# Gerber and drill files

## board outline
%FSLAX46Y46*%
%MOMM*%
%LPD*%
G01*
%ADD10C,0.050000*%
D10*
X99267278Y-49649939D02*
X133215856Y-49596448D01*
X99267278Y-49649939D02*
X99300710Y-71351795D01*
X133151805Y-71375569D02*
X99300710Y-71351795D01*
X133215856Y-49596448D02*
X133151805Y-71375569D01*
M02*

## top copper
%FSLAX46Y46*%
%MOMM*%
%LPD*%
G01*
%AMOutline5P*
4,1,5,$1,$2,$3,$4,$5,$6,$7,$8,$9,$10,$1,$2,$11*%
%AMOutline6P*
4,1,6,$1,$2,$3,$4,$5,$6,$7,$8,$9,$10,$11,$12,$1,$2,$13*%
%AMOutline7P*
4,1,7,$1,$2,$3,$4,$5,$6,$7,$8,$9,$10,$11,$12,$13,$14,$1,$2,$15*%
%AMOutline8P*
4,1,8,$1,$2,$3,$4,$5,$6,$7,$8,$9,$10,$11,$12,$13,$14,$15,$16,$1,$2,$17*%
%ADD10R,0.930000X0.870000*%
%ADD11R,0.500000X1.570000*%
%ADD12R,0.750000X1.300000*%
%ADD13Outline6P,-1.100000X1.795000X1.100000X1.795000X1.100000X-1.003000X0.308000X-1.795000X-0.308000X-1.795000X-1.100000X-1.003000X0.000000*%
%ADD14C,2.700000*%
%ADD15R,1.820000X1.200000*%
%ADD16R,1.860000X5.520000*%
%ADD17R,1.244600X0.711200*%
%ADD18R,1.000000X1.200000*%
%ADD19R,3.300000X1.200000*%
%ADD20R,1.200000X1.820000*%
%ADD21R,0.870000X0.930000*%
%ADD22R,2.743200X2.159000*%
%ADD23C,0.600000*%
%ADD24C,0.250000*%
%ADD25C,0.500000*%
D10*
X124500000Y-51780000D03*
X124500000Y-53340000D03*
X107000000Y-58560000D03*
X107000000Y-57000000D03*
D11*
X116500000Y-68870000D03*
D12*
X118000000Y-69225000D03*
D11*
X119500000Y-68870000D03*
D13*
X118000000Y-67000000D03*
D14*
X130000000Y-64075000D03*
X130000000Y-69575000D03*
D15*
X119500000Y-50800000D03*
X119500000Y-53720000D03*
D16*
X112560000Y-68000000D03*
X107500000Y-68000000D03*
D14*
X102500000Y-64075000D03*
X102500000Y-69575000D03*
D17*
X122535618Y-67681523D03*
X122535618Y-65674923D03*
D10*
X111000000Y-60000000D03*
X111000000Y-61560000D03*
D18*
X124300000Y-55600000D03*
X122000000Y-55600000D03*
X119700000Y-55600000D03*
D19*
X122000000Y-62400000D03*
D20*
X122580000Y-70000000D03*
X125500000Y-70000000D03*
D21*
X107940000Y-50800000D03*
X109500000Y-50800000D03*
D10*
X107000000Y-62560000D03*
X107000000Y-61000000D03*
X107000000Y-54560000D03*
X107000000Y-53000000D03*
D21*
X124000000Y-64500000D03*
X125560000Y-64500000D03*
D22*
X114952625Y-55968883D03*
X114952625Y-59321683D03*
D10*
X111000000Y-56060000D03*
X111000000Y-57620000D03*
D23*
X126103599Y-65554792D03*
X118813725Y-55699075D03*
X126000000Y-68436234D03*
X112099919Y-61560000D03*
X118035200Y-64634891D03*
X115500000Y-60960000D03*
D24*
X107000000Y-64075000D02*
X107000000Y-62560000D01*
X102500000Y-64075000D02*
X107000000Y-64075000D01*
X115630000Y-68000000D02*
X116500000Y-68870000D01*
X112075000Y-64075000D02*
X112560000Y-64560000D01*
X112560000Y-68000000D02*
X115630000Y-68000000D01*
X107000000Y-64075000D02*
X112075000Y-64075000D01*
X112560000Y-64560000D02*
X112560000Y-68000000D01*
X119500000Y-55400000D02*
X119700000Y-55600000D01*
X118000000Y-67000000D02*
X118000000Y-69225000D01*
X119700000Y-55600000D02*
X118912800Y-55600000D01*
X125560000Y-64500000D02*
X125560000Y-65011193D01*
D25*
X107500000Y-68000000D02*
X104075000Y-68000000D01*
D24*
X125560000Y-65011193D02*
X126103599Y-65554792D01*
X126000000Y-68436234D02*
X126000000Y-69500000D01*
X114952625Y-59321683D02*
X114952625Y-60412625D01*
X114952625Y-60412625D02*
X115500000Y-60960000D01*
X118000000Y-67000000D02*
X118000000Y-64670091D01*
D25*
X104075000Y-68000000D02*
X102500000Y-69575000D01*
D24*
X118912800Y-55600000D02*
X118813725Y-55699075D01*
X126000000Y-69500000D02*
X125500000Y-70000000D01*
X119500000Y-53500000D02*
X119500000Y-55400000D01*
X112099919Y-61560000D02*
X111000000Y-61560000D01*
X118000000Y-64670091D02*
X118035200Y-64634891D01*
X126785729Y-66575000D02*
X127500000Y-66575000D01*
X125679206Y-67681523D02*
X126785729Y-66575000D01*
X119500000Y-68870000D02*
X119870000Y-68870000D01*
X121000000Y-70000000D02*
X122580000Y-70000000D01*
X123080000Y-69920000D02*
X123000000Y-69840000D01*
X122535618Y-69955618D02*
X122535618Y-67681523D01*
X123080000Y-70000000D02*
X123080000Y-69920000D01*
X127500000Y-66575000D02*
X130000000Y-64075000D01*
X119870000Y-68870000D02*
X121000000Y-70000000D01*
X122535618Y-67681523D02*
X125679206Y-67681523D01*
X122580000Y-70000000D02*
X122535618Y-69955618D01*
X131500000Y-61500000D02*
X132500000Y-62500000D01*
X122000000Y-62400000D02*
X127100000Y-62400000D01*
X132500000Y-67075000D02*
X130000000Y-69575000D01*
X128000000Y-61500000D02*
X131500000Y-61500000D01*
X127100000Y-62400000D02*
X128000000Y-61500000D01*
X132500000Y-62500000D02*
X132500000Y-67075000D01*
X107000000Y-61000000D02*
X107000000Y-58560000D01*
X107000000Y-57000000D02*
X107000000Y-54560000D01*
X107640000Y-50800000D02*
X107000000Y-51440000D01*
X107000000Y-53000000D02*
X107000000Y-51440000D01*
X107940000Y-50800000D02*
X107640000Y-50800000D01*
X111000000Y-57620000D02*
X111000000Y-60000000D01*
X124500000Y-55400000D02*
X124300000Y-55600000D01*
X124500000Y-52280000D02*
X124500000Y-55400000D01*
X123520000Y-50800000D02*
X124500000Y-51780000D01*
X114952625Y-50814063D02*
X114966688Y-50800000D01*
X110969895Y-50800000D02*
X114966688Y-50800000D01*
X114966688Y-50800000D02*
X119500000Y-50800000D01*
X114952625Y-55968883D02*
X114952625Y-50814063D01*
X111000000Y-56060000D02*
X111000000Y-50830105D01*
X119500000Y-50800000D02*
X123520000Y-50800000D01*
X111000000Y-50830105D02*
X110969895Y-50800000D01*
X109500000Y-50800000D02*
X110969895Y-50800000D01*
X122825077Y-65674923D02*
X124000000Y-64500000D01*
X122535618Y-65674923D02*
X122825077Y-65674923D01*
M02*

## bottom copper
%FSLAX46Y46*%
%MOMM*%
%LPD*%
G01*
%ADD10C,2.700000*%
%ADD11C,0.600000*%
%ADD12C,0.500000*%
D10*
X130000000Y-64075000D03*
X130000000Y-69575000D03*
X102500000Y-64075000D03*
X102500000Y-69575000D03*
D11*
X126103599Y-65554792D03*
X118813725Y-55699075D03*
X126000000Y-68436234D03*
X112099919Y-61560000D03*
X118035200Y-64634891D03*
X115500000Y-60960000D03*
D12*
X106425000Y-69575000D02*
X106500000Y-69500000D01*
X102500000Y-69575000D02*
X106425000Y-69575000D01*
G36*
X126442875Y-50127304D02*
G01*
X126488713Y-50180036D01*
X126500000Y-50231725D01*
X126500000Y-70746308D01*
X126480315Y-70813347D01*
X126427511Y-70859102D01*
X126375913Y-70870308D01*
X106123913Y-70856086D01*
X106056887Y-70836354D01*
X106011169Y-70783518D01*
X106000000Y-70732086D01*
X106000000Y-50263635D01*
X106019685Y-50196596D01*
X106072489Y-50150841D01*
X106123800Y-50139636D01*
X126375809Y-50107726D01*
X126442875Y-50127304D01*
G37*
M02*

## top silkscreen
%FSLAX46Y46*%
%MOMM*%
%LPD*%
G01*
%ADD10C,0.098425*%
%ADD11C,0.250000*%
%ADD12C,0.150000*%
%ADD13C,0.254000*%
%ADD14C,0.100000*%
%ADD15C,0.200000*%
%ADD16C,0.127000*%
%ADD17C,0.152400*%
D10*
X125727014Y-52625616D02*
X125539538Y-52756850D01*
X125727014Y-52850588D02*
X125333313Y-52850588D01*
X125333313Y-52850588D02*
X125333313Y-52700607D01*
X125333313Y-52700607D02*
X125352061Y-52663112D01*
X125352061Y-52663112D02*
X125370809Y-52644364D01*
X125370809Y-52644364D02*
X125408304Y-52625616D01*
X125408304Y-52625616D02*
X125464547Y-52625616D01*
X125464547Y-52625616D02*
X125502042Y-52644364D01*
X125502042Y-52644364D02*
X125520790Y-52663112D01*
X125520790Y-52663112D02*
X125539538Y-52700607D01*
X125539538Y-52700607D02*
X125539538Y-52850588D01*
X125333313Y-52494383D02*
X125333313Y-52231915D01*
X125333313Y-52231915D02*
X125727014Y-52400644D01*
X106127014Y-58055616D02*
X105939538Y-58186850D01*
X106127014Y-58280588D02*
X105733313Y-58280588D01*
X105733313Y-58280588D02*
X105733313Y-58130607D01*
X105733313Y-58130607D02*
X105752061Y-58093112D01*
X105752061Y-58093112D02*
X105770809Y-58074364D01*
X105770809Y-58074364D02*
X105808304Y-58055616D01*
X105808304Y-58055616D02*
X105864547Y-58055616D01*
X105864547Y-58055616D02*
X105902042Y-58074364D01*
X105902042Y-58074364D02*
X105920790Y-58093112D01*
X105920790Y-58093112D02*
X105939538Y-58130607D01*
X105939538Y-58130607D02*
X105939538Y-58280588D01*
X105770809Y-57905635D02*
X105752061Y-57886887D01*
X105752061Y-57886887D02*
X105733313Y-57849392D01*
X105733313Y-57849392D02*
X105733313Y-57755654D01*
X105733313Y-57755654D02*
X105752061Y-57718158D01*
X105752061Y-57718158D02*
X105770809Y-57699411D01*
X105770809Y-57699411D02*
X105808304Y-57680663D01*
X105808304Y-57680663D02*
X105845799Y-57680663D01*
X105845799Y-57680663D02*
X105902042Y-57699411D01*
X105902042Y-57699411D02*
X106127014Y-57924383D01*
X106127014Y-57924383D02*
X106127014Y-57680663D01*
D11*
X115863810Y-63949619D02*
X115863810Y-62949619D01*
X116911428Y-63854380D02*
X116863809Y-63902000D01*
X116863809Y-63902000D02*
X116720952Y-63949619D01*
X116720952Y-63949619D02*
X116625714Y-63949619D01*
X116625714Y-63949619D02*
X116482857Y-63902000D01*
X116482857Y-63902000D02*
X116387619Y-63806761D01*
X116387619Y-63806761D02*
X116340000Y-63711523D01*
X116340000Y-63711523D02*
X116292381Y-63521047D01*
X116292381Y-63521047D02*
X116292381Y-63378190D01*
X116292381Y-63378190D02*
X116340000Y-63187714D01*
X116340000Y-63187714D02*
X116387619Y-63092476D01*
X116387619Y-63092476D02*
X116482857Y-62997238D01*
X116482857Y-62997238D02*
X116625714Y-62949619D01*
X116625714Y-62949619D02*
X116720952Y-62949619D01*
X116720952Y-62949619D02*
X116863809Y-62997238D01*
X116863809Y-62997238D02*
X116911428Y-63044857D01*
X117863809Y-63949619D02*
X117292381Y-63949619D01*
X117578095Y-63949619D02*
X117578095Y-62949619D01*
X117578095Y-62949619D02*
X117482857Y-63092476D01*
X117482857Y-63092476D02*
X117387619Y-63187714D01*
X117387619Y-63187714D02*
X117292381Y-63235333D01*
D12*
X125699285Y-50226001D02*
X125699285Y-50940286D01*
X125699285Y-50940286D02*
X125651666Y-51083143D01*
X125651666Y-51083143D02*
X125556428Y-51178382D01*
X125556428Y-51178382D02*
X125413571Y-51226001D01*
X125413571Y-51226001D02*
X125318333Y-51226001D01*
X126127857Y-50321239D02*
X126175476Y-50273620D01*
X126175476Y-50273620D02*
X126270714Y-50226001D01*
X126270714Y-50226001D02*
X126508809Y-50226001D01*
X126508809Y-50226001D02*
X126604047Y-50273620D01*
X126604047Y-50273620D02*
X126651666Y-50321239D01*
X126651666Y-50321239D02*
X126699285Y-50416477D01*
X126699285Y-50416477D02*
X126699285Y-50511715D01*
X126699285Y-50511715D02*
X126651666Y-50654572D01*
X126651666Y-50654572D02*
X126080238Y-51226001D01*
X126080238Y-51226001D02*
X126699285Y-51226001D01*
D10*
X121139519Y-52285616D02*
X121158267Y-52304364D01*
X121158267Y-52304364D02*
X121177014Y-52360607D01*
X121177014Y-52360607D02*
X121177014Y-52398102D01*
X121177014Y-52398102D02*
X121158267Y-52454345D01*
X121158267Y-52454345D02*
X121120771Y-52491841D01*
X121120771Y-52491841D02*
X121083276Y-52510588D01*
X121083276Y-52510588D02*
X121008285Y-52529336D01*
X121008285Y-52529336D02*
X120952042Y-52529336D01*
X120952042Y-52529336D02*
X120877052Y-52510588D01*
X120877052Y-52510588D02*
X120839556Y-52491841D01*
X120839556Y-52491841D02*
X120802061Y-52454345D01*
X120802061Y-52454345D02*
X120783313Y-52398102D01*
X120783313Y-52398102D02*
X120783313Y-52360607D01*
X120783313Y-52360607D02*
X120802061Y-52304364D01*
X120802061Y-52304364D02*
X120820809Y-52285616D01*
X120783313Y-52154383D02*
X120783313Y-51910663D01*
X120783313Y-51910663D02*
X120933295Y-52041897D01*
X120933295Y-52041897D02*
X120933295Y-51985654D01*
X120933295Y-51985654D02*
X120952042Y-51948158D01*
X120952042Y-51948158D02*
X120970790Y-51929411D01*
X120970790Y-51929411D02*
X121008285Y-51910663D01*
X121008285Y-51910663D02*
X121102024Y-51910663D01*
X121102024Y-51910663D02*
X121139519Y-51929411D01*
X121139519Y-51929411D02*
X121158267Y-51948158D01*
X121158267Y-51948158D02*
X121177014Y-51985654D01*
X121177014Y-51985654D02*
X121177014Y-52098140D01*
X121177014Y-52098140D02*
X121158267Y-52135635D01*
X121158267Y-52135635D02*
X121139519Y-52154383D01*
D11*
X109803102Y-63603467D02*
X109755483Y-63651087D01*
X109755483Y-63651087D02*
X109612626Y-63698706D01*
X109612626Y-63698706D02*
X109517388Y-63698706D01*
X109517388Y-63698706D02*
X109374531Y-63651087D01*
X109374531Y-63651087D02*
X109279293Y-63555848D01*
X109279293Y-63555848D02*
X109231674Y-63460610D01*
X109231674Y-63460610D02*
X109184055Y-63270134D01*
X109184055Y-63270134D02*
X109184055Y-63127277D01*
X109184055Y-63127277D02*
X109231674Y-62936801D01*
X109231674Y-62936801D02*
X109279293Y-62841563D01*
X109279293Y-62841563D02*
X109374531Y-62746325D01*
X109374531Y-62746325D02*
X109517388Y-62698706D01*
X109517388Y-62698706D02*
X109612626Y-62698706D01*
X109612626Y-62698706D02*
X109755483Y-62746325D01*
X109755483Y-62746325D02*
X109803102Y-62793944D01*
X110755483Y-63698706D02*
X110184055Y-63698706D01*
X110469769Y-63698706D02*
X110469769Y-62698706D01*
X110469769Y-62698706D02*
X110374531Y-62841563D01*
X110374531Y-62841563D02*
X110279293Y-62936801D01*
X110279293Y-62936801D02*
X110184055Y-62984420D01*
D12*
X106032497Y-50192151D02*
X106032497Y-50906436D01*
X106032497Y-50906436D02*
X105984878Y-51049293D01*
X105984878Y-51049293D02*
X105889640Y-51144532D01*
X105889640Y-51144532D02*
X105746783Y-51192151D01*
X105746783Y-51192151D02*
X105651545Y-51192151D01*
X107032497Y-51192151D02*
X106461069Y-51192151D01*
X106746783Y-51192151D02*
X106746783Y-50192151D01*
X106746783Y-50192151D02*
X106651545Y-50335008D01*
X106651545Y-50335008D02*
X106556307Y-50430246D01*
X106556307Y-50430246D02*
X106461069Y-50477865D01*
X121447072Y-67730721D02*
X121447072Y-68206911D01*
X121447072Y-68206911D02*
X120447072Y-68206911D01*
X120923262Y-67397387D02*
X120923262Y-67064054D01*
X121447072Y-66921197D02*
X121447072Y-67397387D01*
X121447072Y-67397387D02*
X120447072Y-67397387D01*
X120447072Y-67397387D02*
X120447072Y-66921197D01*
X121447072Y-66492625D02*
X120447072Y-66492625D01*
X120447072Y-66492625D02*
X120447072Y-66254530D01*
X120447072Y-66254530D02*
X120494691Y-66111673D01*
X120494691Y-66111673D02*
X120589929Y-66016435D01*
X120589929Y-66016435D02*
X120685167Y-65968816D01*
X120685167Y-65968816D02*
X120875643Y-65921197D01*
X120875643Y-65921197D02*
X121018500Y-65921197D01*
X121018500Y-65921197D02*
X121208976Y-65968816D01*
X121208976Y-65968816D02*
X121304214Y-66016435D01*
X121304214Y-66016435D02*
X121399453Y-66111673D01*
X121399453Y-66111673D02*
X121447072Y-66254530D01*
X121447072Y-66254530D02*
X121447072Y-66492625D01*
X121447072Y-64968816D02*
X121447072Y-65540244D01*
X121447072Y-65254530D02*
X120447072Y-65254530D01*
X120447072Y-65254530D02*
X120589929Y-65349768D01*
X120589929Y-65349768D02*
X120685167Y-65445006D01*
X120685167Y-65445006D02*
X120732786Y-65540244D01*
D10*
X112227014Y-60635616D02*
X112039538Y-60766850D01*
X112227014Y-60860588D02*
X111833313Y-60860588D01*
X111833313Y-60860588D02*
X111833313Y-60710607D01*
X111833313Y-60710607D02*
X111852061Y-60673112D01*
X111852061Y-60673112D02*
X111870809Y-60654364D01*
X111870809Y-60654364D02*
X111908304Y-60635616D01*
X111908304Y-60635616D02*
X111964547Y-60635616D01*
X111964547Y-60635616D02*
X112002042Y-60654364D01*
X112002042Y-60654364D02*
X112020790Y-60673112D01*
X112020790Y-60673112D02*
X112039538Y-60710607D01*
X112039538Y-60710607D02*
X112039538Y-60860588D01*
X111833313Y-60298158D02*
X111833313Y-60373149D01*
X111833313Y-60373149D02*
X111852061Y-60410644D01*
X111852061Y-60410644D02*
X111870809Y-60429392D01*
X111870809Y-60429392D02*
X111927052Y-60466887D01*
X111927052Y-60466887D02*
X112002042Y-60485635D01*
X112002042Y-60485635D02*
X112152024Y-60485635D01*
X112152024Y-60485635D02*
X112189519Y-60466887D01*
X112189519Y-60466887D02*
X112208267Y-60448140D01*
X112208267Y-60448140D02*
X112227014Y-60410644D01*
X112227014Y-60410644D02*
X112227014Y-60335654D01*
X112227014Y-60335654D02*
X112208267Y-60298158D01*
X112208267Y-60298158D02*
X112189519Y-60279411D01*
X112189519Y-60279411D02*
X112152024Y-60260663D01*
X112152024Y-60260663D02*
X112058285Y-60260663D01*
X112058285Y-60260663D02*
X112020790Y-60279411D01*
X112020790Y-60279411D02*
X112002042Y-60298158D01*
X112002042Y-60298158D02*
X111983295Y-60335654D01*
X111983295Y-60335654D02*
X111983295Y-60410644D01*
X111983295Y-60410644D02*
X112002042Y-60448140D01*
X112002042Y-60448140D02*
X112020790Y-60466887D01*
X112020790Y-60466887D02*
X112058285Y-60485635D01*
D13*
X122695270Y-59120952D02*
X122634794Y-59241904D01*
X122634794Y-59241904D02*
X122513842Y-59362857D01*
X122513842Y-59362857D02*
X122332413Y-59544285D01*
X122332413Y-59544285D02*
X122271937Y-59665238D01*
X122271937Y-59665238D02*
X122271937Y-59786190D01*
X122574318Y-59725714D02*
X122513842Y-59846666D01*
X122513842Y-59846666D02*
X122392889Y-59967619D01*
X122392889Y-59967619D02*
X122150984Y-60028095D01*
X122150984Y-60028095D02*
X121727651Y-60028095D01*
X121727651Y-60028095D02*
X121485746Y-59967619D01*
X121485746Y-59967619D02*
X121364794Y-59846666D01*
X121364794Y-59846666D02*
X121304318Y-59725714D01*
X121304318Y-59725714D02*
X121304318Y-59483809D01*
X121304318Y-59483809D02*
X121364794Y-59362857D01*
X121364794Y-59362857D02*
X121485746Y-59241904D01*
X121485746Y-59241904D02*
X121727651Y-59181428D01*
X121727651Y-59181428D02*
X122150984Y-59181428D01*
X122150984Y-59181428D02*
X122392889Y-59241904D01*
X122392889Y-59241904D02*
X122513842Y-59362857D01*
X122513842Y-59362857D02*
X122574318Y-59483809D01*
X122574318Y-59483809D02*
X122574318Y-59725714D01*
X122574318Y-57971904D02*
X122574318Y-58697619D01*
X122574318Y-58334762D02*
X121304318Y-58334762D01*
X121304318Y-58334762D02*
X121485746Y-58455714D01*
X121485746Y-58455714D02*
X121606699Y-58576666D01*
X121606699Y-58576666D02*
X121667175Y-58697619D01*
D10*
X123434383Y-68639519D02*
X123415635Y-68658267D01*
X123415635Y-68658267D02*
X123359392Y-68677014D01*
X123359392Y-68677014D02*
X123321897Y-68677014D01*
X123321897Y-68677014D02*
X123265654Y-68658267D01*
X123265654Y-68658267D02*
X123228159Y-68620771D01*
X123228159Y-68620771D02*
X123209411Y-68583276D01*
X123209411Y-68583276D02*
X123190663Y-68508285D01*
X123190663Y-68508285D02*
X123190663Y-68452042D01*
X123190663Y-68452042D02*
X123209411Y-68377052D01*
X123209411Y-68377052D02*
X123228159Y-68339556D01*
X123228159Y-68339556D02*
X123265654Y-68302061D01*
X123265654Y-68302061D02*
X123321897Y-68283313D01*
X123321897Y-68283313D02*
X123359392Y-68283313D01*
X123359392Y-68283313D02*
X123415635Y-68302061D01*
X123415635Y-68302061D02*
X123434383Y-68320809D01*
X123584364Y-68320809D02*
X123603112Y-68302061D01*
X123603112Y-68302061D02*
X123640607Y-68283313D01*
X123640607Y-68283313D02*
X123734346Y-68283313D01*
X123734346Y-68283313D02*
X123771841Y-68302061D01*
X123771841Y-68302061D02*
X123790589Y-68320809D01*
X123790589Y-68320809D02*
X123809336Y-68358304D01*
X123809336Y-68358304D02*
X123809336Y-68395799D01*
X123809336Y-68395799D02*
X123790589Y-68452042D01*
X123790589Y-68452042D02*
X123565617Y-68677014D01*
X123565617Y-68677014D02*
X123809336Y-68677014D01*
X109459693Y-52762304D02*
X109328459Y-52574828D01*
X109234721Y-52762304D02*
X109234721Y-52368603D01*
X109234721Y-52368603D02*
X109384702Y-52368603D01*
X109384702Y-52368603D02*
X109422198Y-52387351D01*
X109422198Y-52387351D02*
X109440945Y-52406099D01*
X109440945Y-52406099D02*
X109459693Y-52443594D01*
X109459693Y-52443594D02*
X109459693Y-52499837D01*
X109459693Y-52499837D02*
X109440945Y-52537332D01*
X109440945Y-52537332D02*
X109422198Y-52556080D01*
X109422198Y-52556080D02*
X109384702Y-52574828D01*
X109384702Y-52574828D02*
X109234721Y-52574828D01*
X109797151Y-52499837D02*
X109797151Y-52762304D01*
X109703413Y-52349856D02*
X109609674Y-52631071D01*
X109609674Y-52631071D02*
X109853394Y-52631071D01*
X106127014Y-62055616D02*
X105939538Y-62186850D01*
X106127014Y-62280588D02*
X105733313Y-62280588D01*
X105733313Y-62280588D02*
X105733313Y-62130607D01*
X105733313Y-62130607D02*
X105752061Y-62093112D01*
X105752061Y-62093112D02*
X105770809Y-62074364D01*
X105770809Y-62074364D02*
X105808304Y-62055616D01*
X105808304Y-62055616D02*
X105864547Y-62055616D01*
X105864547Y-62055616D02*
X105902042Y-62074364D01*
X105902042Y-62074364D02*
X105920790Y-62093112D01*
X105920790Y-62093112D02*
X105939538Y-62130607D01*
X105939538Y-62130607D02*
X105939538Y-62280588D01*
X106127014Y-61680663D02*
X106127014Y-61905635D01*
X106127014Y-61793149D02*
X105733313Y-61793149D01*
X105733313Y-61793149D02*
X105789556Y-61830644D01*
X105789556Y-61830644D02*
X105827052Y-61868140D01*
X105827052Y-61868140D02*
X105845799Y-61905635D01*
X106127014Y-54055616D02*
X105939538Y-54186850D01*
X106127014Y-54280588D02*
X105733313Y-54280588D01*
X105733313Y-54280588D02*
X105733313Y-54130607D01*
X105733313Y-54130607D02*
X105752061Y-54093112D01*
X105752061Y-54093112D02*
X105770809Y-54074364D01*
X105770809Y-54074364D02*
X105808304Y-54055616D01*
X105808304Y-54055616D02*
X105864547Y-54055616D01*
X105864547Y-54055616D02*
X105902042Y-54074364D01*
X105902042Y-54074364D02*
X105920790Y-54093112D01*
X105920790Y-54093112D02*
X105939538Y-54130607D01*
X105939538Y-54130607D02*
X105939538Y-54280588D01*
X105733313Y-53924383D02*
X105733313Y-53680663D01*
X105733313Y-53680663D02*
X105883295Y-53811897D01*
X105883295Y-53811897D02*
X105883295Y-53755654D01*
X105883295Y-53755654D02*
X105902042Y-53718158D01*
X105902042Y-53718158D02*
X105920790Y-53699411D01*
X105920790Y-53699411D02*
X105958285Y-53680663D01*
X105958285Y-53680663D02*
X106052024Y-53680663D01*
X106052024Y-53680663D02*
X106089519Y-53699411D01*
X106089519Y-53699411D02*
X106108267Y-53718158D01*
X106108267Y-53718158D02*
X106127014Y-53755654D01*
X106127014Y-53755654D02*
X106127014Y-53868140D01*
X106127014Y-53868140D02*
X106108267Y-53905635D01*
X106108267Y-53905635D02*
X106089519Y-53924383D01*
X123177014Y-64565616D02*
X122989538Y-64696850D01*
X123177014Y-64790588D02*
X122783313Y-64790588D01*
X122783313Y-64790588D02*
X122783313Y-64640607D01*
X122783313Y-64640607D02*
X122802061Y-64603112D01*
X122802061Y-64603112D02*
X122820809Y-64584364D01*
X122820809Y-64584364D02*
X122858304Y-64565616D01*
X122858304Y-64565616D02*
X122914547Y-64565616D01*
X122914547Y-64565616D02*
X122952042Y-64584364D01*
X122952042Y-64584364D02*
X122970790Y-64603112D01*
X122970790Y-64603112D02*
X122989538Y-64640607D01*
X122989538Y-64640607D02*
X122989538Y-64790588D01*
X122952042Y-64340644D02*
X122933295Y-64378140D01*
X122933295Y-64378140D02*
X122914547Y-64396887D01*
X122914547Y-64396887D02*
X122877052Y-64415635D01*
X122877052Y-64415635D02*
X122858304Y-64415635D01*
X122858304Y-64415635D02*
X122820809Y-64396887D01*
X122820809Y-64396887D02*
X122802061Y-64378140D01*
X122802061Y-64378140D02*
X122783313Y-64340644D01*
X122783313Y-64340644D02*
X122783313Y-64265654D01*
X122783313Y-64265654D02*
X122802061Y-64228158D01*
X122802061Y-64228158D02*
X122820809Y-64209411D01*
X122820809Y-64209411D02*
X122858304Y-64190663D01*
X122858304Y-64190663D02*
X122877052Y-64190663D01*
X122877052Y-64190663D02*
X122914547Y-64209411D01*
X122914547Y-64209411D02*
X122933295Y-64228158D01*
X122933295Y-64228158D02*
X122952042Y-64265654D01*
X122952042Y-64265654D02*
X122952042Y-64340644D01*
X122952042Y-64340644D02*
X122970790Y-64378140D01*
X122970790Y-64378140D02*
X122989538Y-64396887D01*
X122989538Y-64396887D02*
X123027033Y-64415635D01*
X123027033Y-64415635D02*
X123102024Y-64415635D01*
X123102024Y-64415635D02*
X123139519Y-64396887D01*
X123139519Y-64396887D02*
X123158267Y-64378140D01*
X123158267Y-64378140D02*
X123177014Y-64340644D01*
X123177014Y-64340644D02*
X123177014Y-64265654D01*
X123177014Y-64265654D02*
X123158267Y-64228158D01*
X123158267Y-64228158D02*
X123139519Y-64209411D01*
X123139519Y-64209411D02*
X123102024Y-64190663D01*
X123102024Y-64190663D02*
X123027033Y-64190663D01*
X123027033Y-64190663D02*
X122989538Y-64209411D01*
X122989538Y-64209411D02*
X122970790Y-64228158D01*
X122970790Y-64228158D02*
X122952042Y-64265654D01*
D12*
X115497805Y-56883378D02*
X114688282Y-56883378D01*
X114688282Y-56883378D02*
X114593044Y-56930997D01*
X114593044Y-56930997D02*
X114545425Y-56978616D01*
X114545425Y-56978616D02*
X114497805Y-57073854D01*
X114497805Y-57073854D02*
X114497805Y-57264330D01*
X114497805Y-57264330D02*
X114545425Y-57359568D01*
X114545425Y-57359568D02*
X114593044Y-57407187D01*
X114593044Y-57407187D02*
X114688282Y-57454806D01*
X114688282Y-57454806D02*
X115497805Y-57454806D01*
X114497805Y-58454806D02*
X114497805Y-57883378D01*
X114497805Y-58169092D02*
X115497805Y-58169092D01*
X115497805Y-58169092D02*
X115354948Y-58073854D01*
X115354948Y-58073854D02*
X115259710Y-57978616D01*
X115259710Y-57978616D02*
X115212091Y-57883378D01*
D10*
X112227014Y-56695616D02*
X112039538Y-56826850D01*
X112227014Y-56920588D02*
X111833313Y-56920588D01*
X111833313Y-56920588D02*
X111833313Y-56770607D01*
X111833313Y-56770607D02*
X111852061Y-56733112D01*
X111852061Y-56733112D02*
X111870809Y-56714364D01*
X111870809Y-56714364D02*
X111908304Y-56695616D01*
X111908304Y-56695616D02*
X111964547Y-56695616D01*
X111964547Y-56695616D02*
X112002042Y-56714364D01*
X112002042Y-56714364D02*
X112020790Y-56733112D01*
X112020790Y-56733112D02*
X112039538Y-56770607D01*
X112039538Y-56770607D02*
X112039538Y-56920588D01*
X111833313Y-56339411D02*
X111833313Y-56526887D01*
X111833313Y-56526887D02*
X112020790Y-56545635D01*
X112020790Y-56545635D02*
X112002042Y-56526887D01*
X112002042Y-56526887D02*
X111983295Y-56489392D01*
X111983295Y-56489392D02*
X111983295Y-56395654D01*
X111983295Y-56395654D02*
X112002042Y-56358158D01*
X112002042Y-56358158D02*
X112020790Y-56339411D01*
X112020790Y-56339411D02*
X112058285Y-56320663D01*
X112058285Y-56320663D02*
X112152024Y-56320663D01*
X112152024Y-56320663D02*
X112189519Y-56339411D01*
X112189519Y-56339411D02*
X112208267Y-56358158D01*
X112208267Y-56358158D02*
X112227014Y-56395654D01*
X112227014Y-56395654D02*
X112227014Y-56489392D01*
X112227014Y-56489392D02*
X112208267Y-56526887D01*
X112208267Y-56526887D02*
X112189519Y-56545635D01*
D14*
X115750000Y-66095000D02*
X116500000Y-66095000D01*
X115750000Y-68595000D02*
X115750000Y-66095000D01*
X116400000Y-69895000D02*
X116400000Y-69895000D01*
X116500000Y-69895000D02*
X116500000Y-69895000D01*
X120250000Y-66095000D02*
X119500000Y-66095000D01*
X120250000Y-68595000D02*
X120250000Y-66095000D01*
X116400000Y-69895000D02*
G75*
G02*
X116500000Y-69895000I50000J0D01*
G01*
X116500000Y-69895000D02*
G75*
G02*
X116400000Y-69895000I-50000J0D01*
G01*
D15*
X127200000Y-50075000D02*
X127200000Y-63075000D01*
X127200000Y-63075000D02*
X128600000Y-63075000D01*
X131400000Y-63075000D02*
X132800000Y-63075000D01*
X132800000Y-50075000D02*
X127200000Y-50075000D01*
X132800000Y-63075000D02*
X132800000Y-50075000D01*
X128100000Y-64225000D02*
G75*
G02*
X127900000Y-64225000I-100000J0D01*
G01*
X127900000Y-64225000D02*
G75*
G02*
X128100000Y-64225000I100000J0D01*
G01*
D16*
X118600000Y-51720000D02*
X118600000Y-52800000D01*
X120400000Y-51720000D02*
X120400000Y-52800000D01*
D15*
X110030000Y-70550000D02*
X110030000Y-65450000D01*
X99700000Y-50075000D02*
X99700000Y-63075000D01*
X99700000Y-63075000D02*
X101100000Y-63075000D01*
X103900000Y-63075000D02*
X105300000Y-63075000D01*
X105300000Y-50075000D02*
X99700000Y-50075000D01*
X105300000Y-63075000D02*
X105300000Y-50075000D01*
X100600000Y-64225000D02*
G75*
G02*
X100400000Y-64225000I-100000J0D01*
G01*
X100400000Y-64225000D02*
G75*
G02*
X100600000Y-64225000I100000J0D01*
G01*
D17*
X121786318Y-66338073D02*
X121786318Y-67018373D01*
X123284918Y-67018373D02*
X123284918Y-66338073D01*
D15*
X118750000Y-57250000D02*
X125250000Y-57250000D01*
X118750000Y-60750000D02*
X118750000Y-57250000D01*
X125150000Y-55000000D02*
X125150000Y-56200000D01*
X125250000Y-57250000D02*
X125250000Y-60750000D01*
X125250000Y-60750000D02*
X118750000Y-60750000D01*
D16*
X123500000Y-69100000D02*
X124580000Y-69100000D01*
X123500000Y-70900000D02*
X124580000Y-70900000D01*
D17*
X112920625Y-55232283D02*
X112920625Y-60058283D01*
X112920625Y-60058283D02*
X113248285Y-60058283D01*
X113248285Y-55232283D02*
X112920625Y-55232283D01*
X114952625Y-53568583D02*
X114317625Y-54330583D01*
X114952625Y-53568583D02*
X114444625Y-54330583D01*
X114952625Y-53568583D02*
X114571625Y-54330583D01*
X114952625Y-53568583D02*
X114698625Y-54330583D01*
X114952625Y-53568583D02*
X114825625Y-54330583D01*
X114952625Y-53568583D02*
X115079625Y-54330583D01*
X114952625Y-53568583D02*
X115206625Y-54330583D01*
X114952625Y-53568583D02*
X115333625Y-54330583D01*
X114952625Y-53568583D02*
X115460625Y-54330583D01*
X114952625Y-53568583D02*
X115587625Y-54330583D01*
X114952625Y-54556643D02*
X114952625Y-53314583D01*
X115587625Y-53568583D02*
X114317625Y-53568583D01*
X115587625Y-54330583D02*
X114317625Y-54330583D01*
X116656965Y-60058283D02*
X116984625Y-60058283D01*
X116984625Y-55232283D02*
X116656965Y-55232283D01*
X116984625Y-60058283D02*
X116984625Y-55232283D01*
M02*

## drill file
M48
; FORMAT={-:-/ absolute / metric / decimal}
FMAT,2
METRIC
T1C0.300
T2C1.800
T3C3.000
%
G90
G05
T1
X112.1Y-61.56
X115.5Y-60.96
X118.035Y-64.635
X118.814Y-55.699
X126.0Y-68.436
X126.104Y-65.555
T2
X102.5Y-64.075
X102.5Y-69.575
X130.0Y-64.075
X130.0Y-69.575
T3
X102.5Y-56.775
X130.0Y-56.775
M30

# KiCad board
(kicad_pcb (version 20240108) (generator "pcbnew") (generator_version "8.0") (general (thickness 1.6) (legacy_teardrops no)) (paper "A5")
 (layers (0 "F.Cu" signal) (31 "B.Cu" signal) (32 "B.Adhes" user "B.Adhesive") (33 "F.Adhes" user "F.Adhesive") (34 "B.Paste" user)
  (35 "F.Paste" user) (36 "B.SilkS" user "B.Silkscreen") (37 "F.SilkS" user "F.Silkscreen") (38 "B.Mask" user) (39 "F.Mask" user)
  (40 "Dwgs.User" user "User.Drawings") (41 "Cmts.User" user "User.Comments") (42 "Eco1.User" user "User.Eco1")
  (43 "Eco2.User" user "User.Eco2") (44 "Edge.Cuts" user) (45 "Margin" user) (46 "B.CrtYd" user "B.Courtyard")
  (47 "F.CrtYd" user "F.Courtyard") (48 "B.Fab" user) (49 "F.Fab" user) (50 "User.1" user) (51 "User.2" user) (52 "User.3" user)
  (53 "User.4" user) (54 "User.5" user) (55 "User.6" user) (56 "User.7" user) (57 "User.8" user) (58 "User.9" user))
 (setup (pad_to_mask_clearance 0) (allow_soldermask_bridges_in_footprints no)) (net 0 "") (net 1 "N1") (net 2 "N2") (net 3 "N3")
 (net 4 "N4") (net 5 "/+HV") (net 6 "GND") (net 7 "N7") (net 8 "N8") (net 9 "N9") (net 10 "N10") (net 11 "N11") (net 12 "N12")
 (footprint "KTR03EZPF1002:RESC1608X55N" (layer "F.Cu") (at 124.5 52.56 -90)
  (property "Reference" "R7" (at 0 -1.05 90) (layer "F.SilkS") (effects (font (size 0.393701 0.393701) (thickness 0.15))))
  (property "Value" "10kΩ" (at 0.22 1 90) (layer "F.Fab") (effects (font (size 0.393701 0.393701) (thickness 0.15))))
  (pad "1" smd rect (at -0.78 0 270) (size 0.87 0.93) (layers "F.Cu" "F.Paste" "F.Mask") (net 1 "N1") (solder_mask_margin 0.102))
  (pad "2" smd rect (at 0.78 0 270) (size 0.87 0.93) (layers "F.Cu" "F.Paste" "F.Mask") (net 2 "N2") (solder_mask_margin 0.102)))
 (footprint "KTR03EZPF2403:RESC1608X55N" (layer "F.Cu") (at 107 57.78 90)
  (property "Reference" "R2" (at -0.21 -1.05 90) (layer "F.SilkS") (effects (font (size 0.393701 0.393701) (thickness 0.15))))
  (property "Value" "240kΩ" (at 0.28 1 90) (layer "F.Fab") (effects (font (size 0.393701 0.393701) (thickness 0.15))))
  (pad "1" smd rect (at -0.78 0 90) (size 0.87 0.93) (layers "F.Cu" "F.Paste" "F.Mask") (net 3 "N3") (solder_mask_margin 0.102))
  (pad "2" smd rect (at 0.78 0 90) (size 0.87 0.93) (layers "F.Cu" "F.Paste" "F.Mask") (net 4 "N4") (solder_mask_margin 0.102)))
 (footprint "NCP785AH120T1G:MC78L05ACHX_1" (layer "F.Cu") (at 118 68.595)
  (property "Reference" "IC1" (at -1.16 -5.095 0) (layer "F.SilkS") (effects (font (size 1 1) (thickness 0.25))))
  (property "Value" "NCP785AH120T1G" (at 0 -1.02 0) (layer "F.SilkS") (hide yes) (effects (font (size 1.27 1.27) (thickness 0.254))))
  (fp_line (start -2.25 -2.5) (end -1.5 -2.5) (stroke (width 0.1) (type solid)) (layer "F.SilkS"))
  (fp_line (start -2.25 0) (end -2.25 -2.5) (stroke (width 0.1) (type solid)) (layer "F.SilkS"))
  (fp_line (start -1.6 1.3) (end -1.6 1.3) (stroke (width 0.1) (type solid)) (layer "F.SilkS"))
  (fp_line (start -1.5 1.3) (end -1.5 1.3) (stroke (width 0.1) (type solid)) (layer "F.SilkS"))
  (fp_line (start 2.25 -2.5) (end 1.5 -2.5) (stroke (width 0.1) (type solid)) (layer "F.SilkS"))
  (fp_line (start 2.25 0) (end 2.25 -2.5) (stroke (width 0.1) (type solid)) (layer "F.SilkS"))
  (fp_arc (start -1.6 1.3) (mid -1.55 1.25) (end -1.5 1.3) (stroke (width 0.1) (type solid)) (layer "F.SilkS"))
  (fp_arc (start -1.5 1.3) (mid -1.55 1.35) (end -1.6 1.3) (stroke (width 0.1) (type solid)) (layer "F.SilkS"))
  (pad "1" smd rect (at -1.5 0.275) (size 0.5 1.57) (layers "F.Cu" "F.Paste" "F.Mask") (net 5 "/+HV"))
  (pad "2" smd rect (at 0 0.63) (size 0.75 1.3) (layers "F.Cu" "F.Paste" "F.Mask") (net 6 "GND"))
  (pad "3" smd rect (at 1.5 0.275) (size 0.5 1.57) (layers "F.Cu" "F.Paste" "F.Mask") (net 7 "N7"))
  (pad "4" smd roundrect (at 0 -1.595) (size 2.2 3.59) (layers "F.Cu" "F.Paste" "F.Mask") (roundrect_rratio 0) (chamfer_ratio 0.36)
   (chamfer bottom_left bottom_right) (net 6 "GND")))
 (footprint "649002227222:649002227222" (layer "F.Cu") (at 130 56.575 180)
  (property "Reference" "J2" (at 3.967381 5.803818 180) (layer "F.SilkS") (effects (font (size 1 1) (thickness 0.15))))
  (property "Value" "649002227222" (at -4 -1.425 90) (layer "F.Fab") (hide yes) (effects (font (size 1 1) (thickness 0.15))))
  (fp_line (start 2.8 6.5) (end 2.8 -6.5) (stroke (width 0.2) (type solid)) (layer "F.SilkS"))
  (fp_line (start 2.8 -6.5) (end 1.4 -6.5) (stroke (width 0.2) (type solid)) (layer "F.SilkS"))
  (fp_line (start -1.4 -6.5) (end -2.8 -6.5) (stroke (width 0.2) (type solid)) (layer "F.SilkS"))
  (fp_line (start -2.8 6.5) (end 2.8 6.5) (stroke (width 0.2) (type solid)) (layer "F.SilkS"))
  (fp_line (start -2.8 -6.5) (end -2.8 6.5) (stroke (width 0.2) (type solid)) (layer "F.SilkS"))
  (fp_circle (center 2 -7.65) (end 2.1 -7.65) (stroke (width 0.2) (type solid)) (fill none) (layer "F.SilkS"))
  (pad "" np_thru_hole circle (at 0 -0.2 180) (size 3 3) (drill 3) (layers "*.Cu" "*.Mask"))
  (pad "1" thru_hole circle (at 0 -7.5 180) (size 2.7 2.7) (drill 1.8) (layers "*.Cu" "*.Mask") (remove_unused_layers no) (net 7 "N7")
   (solder_mask_margin 0.102))
  (pad "2" thru_hole circle (at 0 -13 180) (size 2.7 2.7) (drill 1.8) (layers "*.Cu" "*.Mask") (remove_unused_layers no) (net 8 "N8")
   (solder_mask_margin 0.102)))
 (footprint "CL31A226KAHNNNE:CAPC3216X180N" (layer "F.Cu") (at 119.5 52.26 -90)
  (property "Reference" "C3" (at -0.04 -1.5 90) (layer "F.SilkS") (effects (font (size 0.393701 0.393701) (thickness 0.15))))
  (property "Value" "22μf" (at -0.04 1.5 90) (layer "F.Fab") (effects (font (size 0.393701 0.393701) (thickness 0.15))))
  (fp_line (start -0.54 0.9) (end 0.54 0.9) (stroke (width 0.127) (type solid)) (layer "F.SilkS"))
  (fp_line (start -0.54 -0.9) (end 0.54 -0.9) (stroke (width 0.127) (type solid)) (layer "F.SilkS"))
  (pad "1" smd rect (at -1.46 0 270) (size 1.2 1.82) (layers "F.Cu" "F.Paste" "F.Mask") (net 1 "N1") (solder_mask_margin 0.102))
  (pad "2" smd rect (at 1.46 0 270) (size 1.2 1.82) (layers "F.Cu" "F.Paste" "F.Mask") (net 6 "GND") (solder_mask_margin 0.102)))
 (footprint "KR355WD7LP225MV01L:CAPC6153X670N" (layer "F.Cu") (at 110.03 68 180)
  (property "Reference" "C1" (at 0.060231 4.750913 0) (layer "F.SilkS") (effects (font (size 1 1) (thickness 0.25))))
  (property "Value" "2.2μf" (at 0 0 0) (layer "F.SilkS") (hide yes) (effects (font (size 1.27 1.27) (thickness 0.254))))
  (fp_line (start 0 -2.55) (end 0 2.55) (stroke (width 0.2) (type solid)) (layer "F.SilkS"))
  (pad "1" smd rect (at -2.53 0 180) (size 1.86 5.52) (layers "F.Cu" "F.Paste" "F.Mask") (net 5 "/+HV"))
  (pad "2" smd rect (at 2.53 0 180) (size 1.86 5.52) (layers "F.Cu" "F.Paste" "F.Mask") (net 6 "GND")))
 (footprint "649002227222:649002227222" (layer "F.Cu") (at 102.5 56.575 180)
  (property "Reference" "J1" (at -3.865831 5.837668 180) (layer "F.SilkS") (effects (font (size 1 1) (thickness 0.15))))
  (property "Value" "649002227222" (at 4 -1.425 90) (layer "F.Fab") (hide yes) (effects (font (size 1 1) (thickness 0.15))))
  (fp_line (start 2.8 6.5) (end 2.8 -6.5) (stroke (width 0.2) (type solid)) (layer "F.SilkS"))
  (fp_line (start 2.8 -6.5) (end 1.4 -6.5) (stroke (width 0.2) (type solid)) (layer "F.SilkS"))
  (fp_line (start -1.4 -6.5) (end -2.8 -6.5) (stroke (width 0.2) (type solid)) (layer "F.SilkS"))
  (fp_line (start -2.8 6.5) (end 2.8 6.5) (stroke (width 0.2) (type solid)) (layer "F.SilkS"))
  (fp_line (start -2.8 -6.5) (end -2.8 6.5) (stroke (width 0.2) (type solid)) (layer "F.SilkS"))
  (fp_circle (center 2 -7.65) (end 2.1 -7.65) (stroke (width 0.2) (type solid)) (fill none) (layer "F.SilkS"))
  (pad "" np_thru_hole circle (at 0 -0.2 180) (size 3 3) (drill 3) (layers "*.Cu" "*.Mask"))
  (pad "1" thru_hole circle (at 0 -7.5 180) (size 2.7 2.7) (drill 1.8) (layers "*.Cu" "*.Mask") (remove_unused_layers no) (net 5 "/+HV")
   (solder_mask_margin 0.102))
  (pad "2" thru_hole circle (at 0 -13 180) (size 2.7 2.7) (drill 1.8) (layers "*.Cu" "*.Mask") (remove_unused_layers no) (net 6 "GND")
   (solder_mask_margin 0.102)))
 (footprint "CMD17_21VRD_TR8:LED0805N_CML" (layer "F.Cu") (at 122.535618 66.678223 90)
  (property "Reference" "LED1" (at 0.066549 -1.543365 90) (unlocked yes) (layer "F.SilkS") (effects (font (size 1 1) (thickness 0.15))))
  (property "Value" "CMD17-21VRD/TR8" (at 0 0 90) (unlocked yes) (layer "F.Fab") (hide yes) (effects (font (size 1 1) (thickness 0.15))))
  (fp_line (start 0.34015 -0.7493) (end -0.34015 -0.7493) (stroke (width 0.1524) (type solid)) (layer "F.SilkS"))
  (fp_line (start -0.34015 0.7493) (end 0.34015 0.7493) (stroke (width 0.1524) (type solid)) (layer "F.SilkS"))
  (pad "1" smd rect (at -1.0033 0 90) (size 0.7112 1.2446) (layers "F.Cu" "F.Paste" "F.Mask") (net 7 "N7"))
  (pad "2" smd rect (at 1.0033 0 90) (size 0.7112 1.2446) (layers "F.Cu" "F.Paste" "F.Mask") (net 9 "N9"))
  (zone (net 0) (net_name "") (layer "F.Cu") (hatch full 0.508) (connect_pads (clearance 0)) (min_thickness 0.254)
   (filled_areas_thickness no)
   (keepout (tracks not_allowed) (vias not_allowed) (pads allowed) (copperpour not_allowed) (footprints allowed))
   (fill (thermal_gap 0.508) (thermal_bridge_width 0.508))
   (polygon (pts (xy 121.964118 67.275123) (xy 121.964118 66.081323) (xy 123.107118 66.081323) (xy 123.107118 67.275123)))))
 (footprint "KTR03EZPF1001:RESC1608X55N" (layer "F.Cu") (at 111 60.78 -90)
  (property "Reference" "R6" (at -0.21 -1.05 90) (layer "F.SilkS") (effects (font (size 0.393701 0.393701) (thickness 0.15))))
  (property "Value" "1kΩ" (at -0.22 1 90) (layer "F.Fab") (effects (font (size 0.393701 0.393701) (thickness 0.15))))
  (pad "1" smd rect (at -0.78 0 270) (size 0.87 0.93) (layers "F.Cu" "F.Paste" "F.Mask") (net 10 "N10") (solder_mask_margin 0.102))
  (pad "2" smd rect (at 0.78 0 270) (size 0.87 0.93) (layers "F.Cu" "F.Paste" "F.Mask") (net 6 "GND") (solder_mask_margin 0.102)))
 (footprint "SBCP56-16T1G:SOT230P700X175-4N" (layer "F.Cu") (at 122 59 -90)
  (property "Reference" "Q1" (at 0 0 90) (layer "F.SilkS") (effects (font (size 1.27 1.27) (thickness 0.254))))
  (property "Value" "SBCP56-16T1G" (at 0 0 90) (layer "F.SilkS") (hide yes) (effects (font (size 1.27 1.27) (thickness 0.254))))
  (fp_line (start -1.75 3.25) (end -1.75 -3.25) (stroke (width 0.2) (type solid)) (layer "F.SilkS"))
  (fp_line (start 1.75 3.25) (end -1.75 3.25) (stroke (width 0.2) (type solid)) (layer "F.SilkS"))
  (fp_line (start -4 -3.15) (end -2.8 -3.15) (stroke (width 0.2) (type solid)) (layer "F.SilkS"))
  (fp_line (start -1.75 -3.25) (end 1.75 -3.25) (stroke (width 0.2) (type solid)) (layer "F.SilkS"))
  (fp_line (start 1.75 -3.25) (end 1.75 3.25) (stroke (width 0.2) (type solid)) (layer "F.SilkS"))
  (pad "1" smd rect (at -3.4 -2.3) (size 1 1.2) (layers "F.Cu" "F.Paste" "F.Mask") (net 2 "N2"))
  (pad "2" smd rect (at -3.4 0) (size 1 1.2) (layers "F.Cu" "F.Paste" "F.Mask") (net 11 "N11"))
  (pad "3" smd rect (at -3.4 2.3) (size 1 1.2) (layers "F.Cu" "F.Paste" "F.Mask") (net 6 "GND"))
  (pad "4" smd rect (at 3.4 0 270) (size 1.2 3.3) (layers "F.Cu" "F.Paste" "F.Mask") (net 8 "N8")))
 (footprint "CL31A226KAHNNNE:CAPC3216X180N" (layer "F.Cu") (at 124.04 70)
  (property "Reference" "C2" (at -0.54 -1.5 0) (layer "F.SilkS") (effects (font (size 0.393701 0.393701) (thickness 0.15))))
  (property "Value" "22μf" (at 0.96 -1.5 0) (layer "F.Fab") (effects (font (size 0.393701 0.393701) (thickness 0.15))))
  (fp_line (start -0.54 -0.9) (end 0.54 -0.9) (stroke (width 0.127) (type solid)) (layer "F.SilkS"))
  (fp_line (start -0.54 0.9) (end 0.54 0.9) (stroke (width 0.127) (type solid)) (layer "F.SilkS"))
  (pad "1" smd rect (at -1.46 0) (size 1.2 1.82) (layers "F.Cu" "F.Paste" "F.Mask") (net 7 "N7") (solder_mask_margin 0.102))
  (pad "2" smd rect (at 1.46 0) (size 1.2 1.82) (layers "F.Cu" "F.Paste" "F.Mask") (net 6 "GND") (solder_mask_margin 0.102)))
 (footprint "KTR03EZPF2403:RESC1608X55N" (layer "F.Cu") (at 108.72 50.8)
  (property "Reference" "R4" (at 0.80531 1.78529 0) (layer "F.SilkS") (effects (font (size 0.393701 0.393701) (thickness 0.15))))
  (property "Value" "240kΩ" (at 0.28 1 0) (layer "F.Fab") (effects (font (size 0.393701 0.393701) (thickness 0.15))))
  (pad "1" smd rect (at -0.78 0) (size 0.87 0.93) (layers "F.Cu" "F.Paste" "F.Mask") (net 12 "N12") (solder_mask_margin 0.102))
  (pad "2" smd rect (at 0.78 0) (size 0.87 0.93) (layers "F.Cu" "F.Paste" "F.Mask") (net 1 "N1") (solder_mask_margin 0.102)))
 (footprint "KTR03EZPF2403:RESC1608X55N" (layer "F.Cu") (at 107 61.78 90)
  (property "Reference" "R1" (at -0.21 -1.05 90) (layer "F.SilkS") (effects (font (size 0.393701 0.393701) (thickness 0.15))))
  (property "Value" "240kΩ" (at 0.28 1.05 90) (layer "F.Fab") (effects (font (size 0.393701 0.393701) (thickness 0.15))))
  (pad "1" smd rect (at -0.78 0 90) (size 0.87 0.93) (layers "F.Cu" "F.Paste" "F.Mask") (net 5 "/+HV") (solder_mask_margin 0.102))
  (pad "2" smd rect (at 0.78 0 90) (size 0.87 0.93) (layers "F.Cu" "F.Paste" "F.Mask") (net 3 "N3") (solder_mask_margin 0.102)))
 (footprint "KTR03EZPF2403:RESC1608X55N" (layer "F.Cu") (at 107 53.78 90)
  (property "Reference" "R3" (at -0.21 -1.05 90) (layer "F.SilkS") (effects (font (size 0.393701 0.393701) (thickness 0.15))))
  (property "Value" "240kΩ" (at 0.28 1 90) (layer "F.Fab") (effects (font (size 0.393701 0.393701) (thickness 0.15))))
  (pad "1" smd rect (at -0.78 0 90) (size 0.87 0.93) (layers "F.Cu" "F.Paste" "F.Mask") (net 4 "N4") (solder_mask_margin 0.102))
  (pad "2" smd rect (at 0.78 0 90) (size 0.87 0.93) (layers "F.Cu" "F.Paste" "F.Mask") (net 12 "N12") (solder_mask_margin 0.102)))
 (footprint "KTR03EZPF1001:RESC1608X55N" (layer "F.Cu") (at 124.78 64.5)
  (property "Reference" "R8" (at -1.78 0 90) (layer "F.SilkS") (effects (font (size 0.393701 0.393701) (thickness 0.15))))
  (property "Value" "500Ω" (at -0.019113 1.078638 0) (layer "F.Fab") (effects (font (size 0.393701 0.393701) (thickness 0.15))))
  (pad "1" smd rect (at -0.78 0) (size 0.87 0.93) (layers "F.Cu" "F.Paste" "F.Mask") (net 9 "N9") (solder_mask_margin 0.102))
  (pad "2" smd rect (at 0.78 0) (size 0.87 0.93) (layers "F.Cu" "F.Paste" "F.Mask") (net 6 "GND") (solder_mask_margin 0.102)))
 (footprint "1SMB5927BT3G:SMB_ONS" (layer "F.Cu") (at 114.952625 57.645283 -90)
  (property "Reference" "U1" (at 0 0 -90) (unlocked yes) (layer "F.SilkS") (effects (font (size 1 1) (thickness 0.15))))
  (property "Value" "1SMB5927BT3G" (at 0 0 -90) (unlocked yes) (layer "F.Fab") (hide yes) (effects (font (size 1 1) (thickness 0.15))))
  (fp_line (start -2.413 2.032) (end 2.413 2.032) (stroke (width 0.1524) (type solid)) (layer "F.SilkS"))
  (fp_line (start 2.413 2.032) (end 2.413 1.70434) (stroke (width 0.1524) (type solid)) (layer "F.SilkS"))
  (fp_line (start -2.413 1.70434) (end -2.413 2.032) (stroke (width 0.1524) (type solid)) (layer "F.SilkS"))
  (fp_line (start -4.0767 0) (end -3.3147 0.635) (stroke (width 0.1524) (type solid)) (layer "F.SilkS"))
  (fp_line (start -4.0767 0) (end -3.3147 0.508) (stroke (width 0.1524) (type solid)) (layer "F.SilkS"))
  (fp_line (start -4.0767 0) (end -3.3147 0.381) (stroke (width 0.1524) (type solid)) (layer "F.SilkS"))
  (fp_line (start -4.0767 0) (end -3.3147 0.254) (stroke (width 0.1524) (type solid)) (layer "F.SilkS"))
  (fp_line (start -4.0767 0) (end -3.3147 0.127) (stroke (width 0.1524) (type solid)) (layer "F.SilkS"))
  (fp_line (start -4.0767 0) (end -3.3147 -0.127) (stroke (width 0.1524) (type solid)) (layer "F.SilkS"))
  (fp_line (start -4.0767 0) (end -3.3147 -0.254) (stroke (width 0.1524) (type solid)) (layer "F.SilkS"))
  (fp_line (start -4.0767 0) (end -3.3147 -0.381) (stroke (width 0.1524) (type solid)) (layer "F.SilkS"))
  (fp_line (start -4.0767 0) (end -3.3147 -0.508) (stroke (width 0.1524) (type solid)) (layer "F.SilkS"))
  (fp_line (start -4.0767 0) (end -3.3147 -0.635) (stroke (width 0.1524) (type solid)) (layer "F.SilkS"))
  (fp_line (start -3.08864 0) (end -4.3307 0) (stroke (width 0.1524) (type solid)) (layer "F.SilkS"))
  (fp_line (start -4.0767 -0.635) (end -4.0767 0.635) (stroke (width 0.1524) (type solid)) (layer "F.SilkS"))
  (fp_line (start -3.3147 -0.635) (end -3.3147 0.635) (stroke (width 0.1524) (type solid)) (layer "F.SilkS"))
  (fp_line (start 2.413 -1.70434) (end 2.413 -2.032) (stroke (width 0.1524) (type solid)) (layer "F.SilkS"))
  (fp_line (start -2.413 -2.032) (end -2.413 -1.70434) (stroke (width 0.1524) (type solid)) (layer "F.SilkS"))
  (fp_line (start 2.413 -2.032) (end -2.413 -2.032) (stroke (width 0.1524) (type solid)) (layer "F.SilkS"))
  (pad "1" smd rect (at -1.6764 0 270) (size 2.159 2.7432) (layers "F.Cu" "F.Paste" "F.Mask") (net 1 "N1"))
  (pad "2" smd rect (at 1.6764 0 270) (size 2.159 2.7432) (layers "F.Cu" "F.Paste" "F.Mask") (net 6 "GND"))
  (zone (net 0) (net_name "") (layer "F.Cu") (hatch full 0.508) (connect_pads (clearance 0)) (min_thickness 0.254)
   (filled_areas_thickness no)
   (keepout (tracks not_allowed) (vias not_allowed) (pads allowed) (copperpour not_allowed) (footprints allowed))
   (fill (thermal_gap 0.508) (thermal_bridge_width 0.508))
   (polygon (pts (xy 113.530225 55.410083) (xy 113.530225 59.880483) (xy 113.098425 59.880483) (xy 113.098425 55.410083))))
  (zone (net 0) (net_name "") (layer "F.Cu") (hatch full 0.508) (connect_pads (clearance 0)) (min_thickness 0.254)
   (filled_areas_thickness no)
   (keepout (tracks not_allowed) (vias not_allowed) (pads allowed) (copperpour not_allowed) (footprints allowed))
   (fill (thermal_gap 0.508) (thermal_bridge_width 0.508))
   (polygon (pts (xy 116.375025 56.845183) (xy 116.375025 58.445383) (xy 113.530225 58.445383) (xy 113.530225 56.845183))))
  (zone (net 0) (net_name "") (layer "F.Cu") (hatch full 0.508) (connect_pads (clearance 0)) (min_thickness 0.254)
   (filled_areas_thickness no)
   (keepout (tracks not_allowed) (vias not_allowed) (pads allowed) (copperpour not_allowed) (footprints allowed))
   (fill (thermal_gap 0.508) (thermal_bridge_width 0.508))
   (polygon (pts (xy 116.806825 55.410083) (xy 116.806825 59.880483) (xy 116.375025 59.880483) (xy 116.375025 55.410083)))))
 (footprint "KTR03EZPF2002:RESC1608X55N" (layer "F.Cu") (at 111 56.84 -90)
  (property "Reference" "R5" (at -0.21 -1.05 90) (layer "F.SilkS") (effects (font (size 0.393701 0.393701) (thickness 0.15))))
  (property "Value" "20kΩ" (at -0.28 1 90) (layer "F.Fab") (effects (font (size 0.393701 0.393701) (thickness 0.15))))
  (pad "1" smd rect (at -0.78 0 270) (size 0.87 0.93) (layers "F.Cu" "F.Paste" "F.Mask") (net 1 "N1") (solder_mask_margin 0.102))
  (pad "2" smd rect (at 0.78 0 270) (size 0.87 0.93) (layers "F.Cu" "F.Paste" "F.Mask") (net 10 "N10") (solder_mask_margin 0.102)))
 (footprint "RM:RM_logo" (layer "B.Cu") (at 116.84 55.88 180)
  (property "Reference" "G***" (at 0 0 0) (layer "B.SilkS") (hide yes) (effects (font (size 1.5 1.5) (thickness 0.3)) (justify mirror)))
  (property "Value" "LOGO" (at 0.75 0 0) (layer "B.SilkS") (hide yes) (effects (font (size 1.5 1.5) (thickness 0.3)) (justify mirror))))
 (gr_line (start 99.267278 49.649939) (end 133.215856 49.596448) (stroke (width 0.05) (type default)) (layer "Edge.Cuts"))
 (gr_line (start 99.267278 49.649939) (end 99.30071 71.351795) (stroke (width 0.05) (type default)) (layer "Edge.Cuts"))
 (gr_line (start 133.151805 71.375569) (end 99.30071 71.351795) (stroke (width 0.05) (type default)) (layer "Edge.Cuts"))
 (gr_line (start 133.215856 49.596448) (end 133.151805 71.375569) (stroke (width 0.05) (type default)) (layer "Edge.Cuts"))
 (segment (start 107 64.075) (end 107 62.56) (width 0.25) (layer "F.Cu") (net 5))
 (segment (start 102.5 64.075) (end 107 64.075) (width 0.25) (layer "F.Cu") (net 5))
 (segment (start 115.63 68) (end 116.5 68.87) (width 0.25) (layer "F.Cu") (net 5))
 (segment (start 112.075 64.075) (end 112.56 64.56) (width 0.25) (layer "F.Cu") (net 5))
 (segment (start 112.56 68) (end 115.63 68) (width 0.25) (layer "F.Cu") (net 5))
 (segment (start 107 64.075) (end 112.075 64.075) (width 0.25) (layer "F.Cu") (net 5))
 (segment (start 112.56 64.56) (end 112.56 68) (width 0.25) (layer "F.Cu") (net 5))
 (segment (start 119.5 55.4) (end 119.7 55.6) (width 0.25) (layer "F.Cu") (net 6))
 (segment (start 118 67) (end 118 69.225) (width 0.25) (layer "F.Cu") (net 6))
 (segment (start 119.7 55.6) (end 118.9128 55.6) (width 0.25) (layer "F.Cu") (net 6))
 (segment (start 125.56 64.5) (end 125.56 65.011193) (width 0.25) (layer "F.Cu") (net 6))
 (segment (start 107.5 68) (end 104.075 68) (width 0.5) (layer "F.Cu") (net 6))
 (segment (start 125.56 65.011193) (end 126.103599 65.554792) (width 0.25) (layer "F.Cu") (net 6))
 (segment (start 126 68.436234) (end 126 69.5) (width 0.25) (layer "F.Cu") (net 6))
 (segment (start 114.952625 59.321683) (end 114.952625 60.412625) (width 0.25) (layer "F.Cu") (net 6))
 (segment (start 114.952625 60.412625) (end 115.5 60.96) (width 0.25) (layer "F.Cu") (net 6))
 (segment (start 118 67) (end 118 64.670091) (width 0.25) (layer "F.Cu") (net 6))
 (segment (start 104.075 68) (end 102.5 69.575) (width 0.5) (layer "F.Cu") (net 6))
 (segment (start 118.9128 55.6) (end 118.813725 55.699075) (width 0.25) (layer "F.Cu") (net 6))
 (segment (start 126 69.5) (end 125.5 70) (width 0.25) (layer "F.Cu") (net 6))
 (segment (start 119.5 53.5) (end 119.5 55.4) (width 0.25) (layer "F.Cu") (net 6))
 (segment (start 112.099919 61.56) (end 111 61.56) (width 0.25) (layer "F.Cu") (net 6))
 (segment (start 118 64.670091) (end 118.0352 64.634891) (width 0.25) (layer "F.Cu") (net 6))
 (via (at 126.103599 65.554792) (size 0.6) (drill 0.3) (layers "F.Cu" "B.Cu") (free yes) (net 6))
 (via (at 118.813725 55.699075) (size 0.6) (drill 0.3) (layers "F.Cu" "B.Cu") (free yes) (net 6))
 (via (at 126 68.436234) (size 0.6) (drill 0.3) (layers "F.Cu" "B.Cu") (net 6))
 (via (at 112.099919 61.56) (size 0.6) (drill 0.3) (layers "F.Cu" "B.Cu") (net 6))
 (via (at 118.0352 64.634891) (size 0.6) (drill 0.3) (layers "F.Cu" "B.Cu") (free yes) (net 6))
 (via (at 115.5 60.96) (size 0.6) (drill 0.3) (layers "F.Cu" "B.Cu") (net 6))
 (segment (start 106.425 69.575) (end 106.5 69.5) (width 0.5) (layer "B.Cu") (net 6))
 (segment (start 102.5 69.575) (end 106.425 69.575) (width 0.5) (layer "B.Cu") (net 6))
 (segment (start 126.785729 66.575) (end 127.5 66.575) (width 0.25) (layer "F.Cu") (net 7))
 (segment (start 125.679206 67.681523) (end 126.785729 66.575) (width 0.25) (layer "F.Cu") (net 7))
 (segment (start 119.5 68.87) (end 119.87 68.87) (width 0.25) (layer "F.Cu") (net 7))
 (segment (start 121 70) (end 122.58 70) (width 0.25) (layer "F.Cu") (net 7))
 (segment (start 123.08 69.92) (end 123 69.84) (width 0.25) (layer "F.Cu") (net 7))
 (segment (start 122.535618 69.955618) (end 122.535618 67.681523) (width 0.25) (layer "F.Cu") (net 7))
 (segment (start 123.08 70) (end 123.08 69.92) (width 0.25) (layer "F.Cu") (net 7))
 (segment (start 127.5 66.575) (end 130 64.075) (width 0.25) (layer "F.Cu") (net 7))
 (segment (start 119.87 68.87) (end 121 70) (width 0.25) (layer "F.Cu") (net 7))
 (segment (start 122.535618 67.681523) (end 125.679206 67.681523) (width 0.25) (layer "F.Cu") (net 7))
 (segment (start 122.58 70) (end 122.535618 69.955618) (width 0.25) (layer "F.Cu") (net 7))
 (segment (start 131.5 61.5) (end 132.5 62.5) (width 0.25) (layer "F.Cu") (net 8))
 (segment (start 122 62.4) (end 127.1 62.4) (width 0.25) (layer "F.Cu") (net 8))
 (segment (start 132.5 67.075) (end 130 69.575) (width 0.25) (layer "F.Cu") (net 8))
 (segment (start 128 61.5) (end 131.5 61.5) (width 0.25) (layer "F.Cu") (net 8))
 (segment (start 127.1 62.4) (end 128 61.5) (width 0.25) (layer "F.Cu") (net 8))
 (segment (start 132.5 62.5) (end 132.5 67.075) (width 0.25) (layer "F.Cu") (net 8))
 (segment (start 107 61) (end 107 58.56) (width 0.25) (layer "F.Cu") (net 3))
 (segment (start 107 57) (end 107 54.56) (width 0.25) (layer "F.Cu") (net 4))
 (segment (start 107.64 50.8) (end 107 51.44) (width 0.25) (layer "F.Cu") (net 12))
 (segment (start 107 53) (end 107 51.44) (width 0.25) (layer "F.Cu") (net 12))
 (segment (start 107.94 50.8) (end 107.64 50.8) (width 0.25) (layer "F.Cu") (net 12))
 (segment (start 111 57.62) (end 111 60) (width 0.25) (layer "F.Cu") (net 10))
 (segment (start 124.5 55.4) (end 124.3 55.6) (width 0.25) (layer "F.Cu") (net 2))
 (segment (start 124.5 52.28) (end 124.5 55.4) (width 0.25) (layer "F.Cu") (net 2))
 (segment (start 123.52 50.8) (end 124.5 51.78) (width 0.25) (layer "F.Cu") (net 1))
 (segment (start 114.952625 50.814063) (end 114.966688 50.8) (width 0.25) (layer "F.Cu") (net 1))
 (segment (start 110.969895 50.8) (end 114.966688 50.8) (width 0.25) (layer "F.Cu") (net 1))
 (segment (start 114.966688 50.8) (end 119.5 50.8) (width 0.25) (layer "F.Cu") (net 1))
 (segment (start 114.952625 55.968883) (end 114.952625 50.814063) (width 0.25) (layer "F.Cu") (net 1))
 (segment (start 111 56.06) (end 111 50.830105) (width 0.25) (layer "F.Cu") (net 1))
 (segment (start 119.5 50.8) (end 123.52 50.8) (width 0.25) (layer "F.Cu") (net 1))
 (segment (start 111 50.830105) (end 110.969895 50.8) (width 0.25) (layer "F.Cu") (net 1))
 (segment (start 109.5 50.8) (end 110.969895 50.8) (width 0.25) (layer "F.Cu") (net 1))
 (segment (start 122.825077 65.674923) (end 124 64.5) (width 0.25) (layer "F.Cu") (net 9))
 (segment (start 122.535618 65.674923) (end 122.825077 65.674923) (width 0.25) (layer "F.Cu") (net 9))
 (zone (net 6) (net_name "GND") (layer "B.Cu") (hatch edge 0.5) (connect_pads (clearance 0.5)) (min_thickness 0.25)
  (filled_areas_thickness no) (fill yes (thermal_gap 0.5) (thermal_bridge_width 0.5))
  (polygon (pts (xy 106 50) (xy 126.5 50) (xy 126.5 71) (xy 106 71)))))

